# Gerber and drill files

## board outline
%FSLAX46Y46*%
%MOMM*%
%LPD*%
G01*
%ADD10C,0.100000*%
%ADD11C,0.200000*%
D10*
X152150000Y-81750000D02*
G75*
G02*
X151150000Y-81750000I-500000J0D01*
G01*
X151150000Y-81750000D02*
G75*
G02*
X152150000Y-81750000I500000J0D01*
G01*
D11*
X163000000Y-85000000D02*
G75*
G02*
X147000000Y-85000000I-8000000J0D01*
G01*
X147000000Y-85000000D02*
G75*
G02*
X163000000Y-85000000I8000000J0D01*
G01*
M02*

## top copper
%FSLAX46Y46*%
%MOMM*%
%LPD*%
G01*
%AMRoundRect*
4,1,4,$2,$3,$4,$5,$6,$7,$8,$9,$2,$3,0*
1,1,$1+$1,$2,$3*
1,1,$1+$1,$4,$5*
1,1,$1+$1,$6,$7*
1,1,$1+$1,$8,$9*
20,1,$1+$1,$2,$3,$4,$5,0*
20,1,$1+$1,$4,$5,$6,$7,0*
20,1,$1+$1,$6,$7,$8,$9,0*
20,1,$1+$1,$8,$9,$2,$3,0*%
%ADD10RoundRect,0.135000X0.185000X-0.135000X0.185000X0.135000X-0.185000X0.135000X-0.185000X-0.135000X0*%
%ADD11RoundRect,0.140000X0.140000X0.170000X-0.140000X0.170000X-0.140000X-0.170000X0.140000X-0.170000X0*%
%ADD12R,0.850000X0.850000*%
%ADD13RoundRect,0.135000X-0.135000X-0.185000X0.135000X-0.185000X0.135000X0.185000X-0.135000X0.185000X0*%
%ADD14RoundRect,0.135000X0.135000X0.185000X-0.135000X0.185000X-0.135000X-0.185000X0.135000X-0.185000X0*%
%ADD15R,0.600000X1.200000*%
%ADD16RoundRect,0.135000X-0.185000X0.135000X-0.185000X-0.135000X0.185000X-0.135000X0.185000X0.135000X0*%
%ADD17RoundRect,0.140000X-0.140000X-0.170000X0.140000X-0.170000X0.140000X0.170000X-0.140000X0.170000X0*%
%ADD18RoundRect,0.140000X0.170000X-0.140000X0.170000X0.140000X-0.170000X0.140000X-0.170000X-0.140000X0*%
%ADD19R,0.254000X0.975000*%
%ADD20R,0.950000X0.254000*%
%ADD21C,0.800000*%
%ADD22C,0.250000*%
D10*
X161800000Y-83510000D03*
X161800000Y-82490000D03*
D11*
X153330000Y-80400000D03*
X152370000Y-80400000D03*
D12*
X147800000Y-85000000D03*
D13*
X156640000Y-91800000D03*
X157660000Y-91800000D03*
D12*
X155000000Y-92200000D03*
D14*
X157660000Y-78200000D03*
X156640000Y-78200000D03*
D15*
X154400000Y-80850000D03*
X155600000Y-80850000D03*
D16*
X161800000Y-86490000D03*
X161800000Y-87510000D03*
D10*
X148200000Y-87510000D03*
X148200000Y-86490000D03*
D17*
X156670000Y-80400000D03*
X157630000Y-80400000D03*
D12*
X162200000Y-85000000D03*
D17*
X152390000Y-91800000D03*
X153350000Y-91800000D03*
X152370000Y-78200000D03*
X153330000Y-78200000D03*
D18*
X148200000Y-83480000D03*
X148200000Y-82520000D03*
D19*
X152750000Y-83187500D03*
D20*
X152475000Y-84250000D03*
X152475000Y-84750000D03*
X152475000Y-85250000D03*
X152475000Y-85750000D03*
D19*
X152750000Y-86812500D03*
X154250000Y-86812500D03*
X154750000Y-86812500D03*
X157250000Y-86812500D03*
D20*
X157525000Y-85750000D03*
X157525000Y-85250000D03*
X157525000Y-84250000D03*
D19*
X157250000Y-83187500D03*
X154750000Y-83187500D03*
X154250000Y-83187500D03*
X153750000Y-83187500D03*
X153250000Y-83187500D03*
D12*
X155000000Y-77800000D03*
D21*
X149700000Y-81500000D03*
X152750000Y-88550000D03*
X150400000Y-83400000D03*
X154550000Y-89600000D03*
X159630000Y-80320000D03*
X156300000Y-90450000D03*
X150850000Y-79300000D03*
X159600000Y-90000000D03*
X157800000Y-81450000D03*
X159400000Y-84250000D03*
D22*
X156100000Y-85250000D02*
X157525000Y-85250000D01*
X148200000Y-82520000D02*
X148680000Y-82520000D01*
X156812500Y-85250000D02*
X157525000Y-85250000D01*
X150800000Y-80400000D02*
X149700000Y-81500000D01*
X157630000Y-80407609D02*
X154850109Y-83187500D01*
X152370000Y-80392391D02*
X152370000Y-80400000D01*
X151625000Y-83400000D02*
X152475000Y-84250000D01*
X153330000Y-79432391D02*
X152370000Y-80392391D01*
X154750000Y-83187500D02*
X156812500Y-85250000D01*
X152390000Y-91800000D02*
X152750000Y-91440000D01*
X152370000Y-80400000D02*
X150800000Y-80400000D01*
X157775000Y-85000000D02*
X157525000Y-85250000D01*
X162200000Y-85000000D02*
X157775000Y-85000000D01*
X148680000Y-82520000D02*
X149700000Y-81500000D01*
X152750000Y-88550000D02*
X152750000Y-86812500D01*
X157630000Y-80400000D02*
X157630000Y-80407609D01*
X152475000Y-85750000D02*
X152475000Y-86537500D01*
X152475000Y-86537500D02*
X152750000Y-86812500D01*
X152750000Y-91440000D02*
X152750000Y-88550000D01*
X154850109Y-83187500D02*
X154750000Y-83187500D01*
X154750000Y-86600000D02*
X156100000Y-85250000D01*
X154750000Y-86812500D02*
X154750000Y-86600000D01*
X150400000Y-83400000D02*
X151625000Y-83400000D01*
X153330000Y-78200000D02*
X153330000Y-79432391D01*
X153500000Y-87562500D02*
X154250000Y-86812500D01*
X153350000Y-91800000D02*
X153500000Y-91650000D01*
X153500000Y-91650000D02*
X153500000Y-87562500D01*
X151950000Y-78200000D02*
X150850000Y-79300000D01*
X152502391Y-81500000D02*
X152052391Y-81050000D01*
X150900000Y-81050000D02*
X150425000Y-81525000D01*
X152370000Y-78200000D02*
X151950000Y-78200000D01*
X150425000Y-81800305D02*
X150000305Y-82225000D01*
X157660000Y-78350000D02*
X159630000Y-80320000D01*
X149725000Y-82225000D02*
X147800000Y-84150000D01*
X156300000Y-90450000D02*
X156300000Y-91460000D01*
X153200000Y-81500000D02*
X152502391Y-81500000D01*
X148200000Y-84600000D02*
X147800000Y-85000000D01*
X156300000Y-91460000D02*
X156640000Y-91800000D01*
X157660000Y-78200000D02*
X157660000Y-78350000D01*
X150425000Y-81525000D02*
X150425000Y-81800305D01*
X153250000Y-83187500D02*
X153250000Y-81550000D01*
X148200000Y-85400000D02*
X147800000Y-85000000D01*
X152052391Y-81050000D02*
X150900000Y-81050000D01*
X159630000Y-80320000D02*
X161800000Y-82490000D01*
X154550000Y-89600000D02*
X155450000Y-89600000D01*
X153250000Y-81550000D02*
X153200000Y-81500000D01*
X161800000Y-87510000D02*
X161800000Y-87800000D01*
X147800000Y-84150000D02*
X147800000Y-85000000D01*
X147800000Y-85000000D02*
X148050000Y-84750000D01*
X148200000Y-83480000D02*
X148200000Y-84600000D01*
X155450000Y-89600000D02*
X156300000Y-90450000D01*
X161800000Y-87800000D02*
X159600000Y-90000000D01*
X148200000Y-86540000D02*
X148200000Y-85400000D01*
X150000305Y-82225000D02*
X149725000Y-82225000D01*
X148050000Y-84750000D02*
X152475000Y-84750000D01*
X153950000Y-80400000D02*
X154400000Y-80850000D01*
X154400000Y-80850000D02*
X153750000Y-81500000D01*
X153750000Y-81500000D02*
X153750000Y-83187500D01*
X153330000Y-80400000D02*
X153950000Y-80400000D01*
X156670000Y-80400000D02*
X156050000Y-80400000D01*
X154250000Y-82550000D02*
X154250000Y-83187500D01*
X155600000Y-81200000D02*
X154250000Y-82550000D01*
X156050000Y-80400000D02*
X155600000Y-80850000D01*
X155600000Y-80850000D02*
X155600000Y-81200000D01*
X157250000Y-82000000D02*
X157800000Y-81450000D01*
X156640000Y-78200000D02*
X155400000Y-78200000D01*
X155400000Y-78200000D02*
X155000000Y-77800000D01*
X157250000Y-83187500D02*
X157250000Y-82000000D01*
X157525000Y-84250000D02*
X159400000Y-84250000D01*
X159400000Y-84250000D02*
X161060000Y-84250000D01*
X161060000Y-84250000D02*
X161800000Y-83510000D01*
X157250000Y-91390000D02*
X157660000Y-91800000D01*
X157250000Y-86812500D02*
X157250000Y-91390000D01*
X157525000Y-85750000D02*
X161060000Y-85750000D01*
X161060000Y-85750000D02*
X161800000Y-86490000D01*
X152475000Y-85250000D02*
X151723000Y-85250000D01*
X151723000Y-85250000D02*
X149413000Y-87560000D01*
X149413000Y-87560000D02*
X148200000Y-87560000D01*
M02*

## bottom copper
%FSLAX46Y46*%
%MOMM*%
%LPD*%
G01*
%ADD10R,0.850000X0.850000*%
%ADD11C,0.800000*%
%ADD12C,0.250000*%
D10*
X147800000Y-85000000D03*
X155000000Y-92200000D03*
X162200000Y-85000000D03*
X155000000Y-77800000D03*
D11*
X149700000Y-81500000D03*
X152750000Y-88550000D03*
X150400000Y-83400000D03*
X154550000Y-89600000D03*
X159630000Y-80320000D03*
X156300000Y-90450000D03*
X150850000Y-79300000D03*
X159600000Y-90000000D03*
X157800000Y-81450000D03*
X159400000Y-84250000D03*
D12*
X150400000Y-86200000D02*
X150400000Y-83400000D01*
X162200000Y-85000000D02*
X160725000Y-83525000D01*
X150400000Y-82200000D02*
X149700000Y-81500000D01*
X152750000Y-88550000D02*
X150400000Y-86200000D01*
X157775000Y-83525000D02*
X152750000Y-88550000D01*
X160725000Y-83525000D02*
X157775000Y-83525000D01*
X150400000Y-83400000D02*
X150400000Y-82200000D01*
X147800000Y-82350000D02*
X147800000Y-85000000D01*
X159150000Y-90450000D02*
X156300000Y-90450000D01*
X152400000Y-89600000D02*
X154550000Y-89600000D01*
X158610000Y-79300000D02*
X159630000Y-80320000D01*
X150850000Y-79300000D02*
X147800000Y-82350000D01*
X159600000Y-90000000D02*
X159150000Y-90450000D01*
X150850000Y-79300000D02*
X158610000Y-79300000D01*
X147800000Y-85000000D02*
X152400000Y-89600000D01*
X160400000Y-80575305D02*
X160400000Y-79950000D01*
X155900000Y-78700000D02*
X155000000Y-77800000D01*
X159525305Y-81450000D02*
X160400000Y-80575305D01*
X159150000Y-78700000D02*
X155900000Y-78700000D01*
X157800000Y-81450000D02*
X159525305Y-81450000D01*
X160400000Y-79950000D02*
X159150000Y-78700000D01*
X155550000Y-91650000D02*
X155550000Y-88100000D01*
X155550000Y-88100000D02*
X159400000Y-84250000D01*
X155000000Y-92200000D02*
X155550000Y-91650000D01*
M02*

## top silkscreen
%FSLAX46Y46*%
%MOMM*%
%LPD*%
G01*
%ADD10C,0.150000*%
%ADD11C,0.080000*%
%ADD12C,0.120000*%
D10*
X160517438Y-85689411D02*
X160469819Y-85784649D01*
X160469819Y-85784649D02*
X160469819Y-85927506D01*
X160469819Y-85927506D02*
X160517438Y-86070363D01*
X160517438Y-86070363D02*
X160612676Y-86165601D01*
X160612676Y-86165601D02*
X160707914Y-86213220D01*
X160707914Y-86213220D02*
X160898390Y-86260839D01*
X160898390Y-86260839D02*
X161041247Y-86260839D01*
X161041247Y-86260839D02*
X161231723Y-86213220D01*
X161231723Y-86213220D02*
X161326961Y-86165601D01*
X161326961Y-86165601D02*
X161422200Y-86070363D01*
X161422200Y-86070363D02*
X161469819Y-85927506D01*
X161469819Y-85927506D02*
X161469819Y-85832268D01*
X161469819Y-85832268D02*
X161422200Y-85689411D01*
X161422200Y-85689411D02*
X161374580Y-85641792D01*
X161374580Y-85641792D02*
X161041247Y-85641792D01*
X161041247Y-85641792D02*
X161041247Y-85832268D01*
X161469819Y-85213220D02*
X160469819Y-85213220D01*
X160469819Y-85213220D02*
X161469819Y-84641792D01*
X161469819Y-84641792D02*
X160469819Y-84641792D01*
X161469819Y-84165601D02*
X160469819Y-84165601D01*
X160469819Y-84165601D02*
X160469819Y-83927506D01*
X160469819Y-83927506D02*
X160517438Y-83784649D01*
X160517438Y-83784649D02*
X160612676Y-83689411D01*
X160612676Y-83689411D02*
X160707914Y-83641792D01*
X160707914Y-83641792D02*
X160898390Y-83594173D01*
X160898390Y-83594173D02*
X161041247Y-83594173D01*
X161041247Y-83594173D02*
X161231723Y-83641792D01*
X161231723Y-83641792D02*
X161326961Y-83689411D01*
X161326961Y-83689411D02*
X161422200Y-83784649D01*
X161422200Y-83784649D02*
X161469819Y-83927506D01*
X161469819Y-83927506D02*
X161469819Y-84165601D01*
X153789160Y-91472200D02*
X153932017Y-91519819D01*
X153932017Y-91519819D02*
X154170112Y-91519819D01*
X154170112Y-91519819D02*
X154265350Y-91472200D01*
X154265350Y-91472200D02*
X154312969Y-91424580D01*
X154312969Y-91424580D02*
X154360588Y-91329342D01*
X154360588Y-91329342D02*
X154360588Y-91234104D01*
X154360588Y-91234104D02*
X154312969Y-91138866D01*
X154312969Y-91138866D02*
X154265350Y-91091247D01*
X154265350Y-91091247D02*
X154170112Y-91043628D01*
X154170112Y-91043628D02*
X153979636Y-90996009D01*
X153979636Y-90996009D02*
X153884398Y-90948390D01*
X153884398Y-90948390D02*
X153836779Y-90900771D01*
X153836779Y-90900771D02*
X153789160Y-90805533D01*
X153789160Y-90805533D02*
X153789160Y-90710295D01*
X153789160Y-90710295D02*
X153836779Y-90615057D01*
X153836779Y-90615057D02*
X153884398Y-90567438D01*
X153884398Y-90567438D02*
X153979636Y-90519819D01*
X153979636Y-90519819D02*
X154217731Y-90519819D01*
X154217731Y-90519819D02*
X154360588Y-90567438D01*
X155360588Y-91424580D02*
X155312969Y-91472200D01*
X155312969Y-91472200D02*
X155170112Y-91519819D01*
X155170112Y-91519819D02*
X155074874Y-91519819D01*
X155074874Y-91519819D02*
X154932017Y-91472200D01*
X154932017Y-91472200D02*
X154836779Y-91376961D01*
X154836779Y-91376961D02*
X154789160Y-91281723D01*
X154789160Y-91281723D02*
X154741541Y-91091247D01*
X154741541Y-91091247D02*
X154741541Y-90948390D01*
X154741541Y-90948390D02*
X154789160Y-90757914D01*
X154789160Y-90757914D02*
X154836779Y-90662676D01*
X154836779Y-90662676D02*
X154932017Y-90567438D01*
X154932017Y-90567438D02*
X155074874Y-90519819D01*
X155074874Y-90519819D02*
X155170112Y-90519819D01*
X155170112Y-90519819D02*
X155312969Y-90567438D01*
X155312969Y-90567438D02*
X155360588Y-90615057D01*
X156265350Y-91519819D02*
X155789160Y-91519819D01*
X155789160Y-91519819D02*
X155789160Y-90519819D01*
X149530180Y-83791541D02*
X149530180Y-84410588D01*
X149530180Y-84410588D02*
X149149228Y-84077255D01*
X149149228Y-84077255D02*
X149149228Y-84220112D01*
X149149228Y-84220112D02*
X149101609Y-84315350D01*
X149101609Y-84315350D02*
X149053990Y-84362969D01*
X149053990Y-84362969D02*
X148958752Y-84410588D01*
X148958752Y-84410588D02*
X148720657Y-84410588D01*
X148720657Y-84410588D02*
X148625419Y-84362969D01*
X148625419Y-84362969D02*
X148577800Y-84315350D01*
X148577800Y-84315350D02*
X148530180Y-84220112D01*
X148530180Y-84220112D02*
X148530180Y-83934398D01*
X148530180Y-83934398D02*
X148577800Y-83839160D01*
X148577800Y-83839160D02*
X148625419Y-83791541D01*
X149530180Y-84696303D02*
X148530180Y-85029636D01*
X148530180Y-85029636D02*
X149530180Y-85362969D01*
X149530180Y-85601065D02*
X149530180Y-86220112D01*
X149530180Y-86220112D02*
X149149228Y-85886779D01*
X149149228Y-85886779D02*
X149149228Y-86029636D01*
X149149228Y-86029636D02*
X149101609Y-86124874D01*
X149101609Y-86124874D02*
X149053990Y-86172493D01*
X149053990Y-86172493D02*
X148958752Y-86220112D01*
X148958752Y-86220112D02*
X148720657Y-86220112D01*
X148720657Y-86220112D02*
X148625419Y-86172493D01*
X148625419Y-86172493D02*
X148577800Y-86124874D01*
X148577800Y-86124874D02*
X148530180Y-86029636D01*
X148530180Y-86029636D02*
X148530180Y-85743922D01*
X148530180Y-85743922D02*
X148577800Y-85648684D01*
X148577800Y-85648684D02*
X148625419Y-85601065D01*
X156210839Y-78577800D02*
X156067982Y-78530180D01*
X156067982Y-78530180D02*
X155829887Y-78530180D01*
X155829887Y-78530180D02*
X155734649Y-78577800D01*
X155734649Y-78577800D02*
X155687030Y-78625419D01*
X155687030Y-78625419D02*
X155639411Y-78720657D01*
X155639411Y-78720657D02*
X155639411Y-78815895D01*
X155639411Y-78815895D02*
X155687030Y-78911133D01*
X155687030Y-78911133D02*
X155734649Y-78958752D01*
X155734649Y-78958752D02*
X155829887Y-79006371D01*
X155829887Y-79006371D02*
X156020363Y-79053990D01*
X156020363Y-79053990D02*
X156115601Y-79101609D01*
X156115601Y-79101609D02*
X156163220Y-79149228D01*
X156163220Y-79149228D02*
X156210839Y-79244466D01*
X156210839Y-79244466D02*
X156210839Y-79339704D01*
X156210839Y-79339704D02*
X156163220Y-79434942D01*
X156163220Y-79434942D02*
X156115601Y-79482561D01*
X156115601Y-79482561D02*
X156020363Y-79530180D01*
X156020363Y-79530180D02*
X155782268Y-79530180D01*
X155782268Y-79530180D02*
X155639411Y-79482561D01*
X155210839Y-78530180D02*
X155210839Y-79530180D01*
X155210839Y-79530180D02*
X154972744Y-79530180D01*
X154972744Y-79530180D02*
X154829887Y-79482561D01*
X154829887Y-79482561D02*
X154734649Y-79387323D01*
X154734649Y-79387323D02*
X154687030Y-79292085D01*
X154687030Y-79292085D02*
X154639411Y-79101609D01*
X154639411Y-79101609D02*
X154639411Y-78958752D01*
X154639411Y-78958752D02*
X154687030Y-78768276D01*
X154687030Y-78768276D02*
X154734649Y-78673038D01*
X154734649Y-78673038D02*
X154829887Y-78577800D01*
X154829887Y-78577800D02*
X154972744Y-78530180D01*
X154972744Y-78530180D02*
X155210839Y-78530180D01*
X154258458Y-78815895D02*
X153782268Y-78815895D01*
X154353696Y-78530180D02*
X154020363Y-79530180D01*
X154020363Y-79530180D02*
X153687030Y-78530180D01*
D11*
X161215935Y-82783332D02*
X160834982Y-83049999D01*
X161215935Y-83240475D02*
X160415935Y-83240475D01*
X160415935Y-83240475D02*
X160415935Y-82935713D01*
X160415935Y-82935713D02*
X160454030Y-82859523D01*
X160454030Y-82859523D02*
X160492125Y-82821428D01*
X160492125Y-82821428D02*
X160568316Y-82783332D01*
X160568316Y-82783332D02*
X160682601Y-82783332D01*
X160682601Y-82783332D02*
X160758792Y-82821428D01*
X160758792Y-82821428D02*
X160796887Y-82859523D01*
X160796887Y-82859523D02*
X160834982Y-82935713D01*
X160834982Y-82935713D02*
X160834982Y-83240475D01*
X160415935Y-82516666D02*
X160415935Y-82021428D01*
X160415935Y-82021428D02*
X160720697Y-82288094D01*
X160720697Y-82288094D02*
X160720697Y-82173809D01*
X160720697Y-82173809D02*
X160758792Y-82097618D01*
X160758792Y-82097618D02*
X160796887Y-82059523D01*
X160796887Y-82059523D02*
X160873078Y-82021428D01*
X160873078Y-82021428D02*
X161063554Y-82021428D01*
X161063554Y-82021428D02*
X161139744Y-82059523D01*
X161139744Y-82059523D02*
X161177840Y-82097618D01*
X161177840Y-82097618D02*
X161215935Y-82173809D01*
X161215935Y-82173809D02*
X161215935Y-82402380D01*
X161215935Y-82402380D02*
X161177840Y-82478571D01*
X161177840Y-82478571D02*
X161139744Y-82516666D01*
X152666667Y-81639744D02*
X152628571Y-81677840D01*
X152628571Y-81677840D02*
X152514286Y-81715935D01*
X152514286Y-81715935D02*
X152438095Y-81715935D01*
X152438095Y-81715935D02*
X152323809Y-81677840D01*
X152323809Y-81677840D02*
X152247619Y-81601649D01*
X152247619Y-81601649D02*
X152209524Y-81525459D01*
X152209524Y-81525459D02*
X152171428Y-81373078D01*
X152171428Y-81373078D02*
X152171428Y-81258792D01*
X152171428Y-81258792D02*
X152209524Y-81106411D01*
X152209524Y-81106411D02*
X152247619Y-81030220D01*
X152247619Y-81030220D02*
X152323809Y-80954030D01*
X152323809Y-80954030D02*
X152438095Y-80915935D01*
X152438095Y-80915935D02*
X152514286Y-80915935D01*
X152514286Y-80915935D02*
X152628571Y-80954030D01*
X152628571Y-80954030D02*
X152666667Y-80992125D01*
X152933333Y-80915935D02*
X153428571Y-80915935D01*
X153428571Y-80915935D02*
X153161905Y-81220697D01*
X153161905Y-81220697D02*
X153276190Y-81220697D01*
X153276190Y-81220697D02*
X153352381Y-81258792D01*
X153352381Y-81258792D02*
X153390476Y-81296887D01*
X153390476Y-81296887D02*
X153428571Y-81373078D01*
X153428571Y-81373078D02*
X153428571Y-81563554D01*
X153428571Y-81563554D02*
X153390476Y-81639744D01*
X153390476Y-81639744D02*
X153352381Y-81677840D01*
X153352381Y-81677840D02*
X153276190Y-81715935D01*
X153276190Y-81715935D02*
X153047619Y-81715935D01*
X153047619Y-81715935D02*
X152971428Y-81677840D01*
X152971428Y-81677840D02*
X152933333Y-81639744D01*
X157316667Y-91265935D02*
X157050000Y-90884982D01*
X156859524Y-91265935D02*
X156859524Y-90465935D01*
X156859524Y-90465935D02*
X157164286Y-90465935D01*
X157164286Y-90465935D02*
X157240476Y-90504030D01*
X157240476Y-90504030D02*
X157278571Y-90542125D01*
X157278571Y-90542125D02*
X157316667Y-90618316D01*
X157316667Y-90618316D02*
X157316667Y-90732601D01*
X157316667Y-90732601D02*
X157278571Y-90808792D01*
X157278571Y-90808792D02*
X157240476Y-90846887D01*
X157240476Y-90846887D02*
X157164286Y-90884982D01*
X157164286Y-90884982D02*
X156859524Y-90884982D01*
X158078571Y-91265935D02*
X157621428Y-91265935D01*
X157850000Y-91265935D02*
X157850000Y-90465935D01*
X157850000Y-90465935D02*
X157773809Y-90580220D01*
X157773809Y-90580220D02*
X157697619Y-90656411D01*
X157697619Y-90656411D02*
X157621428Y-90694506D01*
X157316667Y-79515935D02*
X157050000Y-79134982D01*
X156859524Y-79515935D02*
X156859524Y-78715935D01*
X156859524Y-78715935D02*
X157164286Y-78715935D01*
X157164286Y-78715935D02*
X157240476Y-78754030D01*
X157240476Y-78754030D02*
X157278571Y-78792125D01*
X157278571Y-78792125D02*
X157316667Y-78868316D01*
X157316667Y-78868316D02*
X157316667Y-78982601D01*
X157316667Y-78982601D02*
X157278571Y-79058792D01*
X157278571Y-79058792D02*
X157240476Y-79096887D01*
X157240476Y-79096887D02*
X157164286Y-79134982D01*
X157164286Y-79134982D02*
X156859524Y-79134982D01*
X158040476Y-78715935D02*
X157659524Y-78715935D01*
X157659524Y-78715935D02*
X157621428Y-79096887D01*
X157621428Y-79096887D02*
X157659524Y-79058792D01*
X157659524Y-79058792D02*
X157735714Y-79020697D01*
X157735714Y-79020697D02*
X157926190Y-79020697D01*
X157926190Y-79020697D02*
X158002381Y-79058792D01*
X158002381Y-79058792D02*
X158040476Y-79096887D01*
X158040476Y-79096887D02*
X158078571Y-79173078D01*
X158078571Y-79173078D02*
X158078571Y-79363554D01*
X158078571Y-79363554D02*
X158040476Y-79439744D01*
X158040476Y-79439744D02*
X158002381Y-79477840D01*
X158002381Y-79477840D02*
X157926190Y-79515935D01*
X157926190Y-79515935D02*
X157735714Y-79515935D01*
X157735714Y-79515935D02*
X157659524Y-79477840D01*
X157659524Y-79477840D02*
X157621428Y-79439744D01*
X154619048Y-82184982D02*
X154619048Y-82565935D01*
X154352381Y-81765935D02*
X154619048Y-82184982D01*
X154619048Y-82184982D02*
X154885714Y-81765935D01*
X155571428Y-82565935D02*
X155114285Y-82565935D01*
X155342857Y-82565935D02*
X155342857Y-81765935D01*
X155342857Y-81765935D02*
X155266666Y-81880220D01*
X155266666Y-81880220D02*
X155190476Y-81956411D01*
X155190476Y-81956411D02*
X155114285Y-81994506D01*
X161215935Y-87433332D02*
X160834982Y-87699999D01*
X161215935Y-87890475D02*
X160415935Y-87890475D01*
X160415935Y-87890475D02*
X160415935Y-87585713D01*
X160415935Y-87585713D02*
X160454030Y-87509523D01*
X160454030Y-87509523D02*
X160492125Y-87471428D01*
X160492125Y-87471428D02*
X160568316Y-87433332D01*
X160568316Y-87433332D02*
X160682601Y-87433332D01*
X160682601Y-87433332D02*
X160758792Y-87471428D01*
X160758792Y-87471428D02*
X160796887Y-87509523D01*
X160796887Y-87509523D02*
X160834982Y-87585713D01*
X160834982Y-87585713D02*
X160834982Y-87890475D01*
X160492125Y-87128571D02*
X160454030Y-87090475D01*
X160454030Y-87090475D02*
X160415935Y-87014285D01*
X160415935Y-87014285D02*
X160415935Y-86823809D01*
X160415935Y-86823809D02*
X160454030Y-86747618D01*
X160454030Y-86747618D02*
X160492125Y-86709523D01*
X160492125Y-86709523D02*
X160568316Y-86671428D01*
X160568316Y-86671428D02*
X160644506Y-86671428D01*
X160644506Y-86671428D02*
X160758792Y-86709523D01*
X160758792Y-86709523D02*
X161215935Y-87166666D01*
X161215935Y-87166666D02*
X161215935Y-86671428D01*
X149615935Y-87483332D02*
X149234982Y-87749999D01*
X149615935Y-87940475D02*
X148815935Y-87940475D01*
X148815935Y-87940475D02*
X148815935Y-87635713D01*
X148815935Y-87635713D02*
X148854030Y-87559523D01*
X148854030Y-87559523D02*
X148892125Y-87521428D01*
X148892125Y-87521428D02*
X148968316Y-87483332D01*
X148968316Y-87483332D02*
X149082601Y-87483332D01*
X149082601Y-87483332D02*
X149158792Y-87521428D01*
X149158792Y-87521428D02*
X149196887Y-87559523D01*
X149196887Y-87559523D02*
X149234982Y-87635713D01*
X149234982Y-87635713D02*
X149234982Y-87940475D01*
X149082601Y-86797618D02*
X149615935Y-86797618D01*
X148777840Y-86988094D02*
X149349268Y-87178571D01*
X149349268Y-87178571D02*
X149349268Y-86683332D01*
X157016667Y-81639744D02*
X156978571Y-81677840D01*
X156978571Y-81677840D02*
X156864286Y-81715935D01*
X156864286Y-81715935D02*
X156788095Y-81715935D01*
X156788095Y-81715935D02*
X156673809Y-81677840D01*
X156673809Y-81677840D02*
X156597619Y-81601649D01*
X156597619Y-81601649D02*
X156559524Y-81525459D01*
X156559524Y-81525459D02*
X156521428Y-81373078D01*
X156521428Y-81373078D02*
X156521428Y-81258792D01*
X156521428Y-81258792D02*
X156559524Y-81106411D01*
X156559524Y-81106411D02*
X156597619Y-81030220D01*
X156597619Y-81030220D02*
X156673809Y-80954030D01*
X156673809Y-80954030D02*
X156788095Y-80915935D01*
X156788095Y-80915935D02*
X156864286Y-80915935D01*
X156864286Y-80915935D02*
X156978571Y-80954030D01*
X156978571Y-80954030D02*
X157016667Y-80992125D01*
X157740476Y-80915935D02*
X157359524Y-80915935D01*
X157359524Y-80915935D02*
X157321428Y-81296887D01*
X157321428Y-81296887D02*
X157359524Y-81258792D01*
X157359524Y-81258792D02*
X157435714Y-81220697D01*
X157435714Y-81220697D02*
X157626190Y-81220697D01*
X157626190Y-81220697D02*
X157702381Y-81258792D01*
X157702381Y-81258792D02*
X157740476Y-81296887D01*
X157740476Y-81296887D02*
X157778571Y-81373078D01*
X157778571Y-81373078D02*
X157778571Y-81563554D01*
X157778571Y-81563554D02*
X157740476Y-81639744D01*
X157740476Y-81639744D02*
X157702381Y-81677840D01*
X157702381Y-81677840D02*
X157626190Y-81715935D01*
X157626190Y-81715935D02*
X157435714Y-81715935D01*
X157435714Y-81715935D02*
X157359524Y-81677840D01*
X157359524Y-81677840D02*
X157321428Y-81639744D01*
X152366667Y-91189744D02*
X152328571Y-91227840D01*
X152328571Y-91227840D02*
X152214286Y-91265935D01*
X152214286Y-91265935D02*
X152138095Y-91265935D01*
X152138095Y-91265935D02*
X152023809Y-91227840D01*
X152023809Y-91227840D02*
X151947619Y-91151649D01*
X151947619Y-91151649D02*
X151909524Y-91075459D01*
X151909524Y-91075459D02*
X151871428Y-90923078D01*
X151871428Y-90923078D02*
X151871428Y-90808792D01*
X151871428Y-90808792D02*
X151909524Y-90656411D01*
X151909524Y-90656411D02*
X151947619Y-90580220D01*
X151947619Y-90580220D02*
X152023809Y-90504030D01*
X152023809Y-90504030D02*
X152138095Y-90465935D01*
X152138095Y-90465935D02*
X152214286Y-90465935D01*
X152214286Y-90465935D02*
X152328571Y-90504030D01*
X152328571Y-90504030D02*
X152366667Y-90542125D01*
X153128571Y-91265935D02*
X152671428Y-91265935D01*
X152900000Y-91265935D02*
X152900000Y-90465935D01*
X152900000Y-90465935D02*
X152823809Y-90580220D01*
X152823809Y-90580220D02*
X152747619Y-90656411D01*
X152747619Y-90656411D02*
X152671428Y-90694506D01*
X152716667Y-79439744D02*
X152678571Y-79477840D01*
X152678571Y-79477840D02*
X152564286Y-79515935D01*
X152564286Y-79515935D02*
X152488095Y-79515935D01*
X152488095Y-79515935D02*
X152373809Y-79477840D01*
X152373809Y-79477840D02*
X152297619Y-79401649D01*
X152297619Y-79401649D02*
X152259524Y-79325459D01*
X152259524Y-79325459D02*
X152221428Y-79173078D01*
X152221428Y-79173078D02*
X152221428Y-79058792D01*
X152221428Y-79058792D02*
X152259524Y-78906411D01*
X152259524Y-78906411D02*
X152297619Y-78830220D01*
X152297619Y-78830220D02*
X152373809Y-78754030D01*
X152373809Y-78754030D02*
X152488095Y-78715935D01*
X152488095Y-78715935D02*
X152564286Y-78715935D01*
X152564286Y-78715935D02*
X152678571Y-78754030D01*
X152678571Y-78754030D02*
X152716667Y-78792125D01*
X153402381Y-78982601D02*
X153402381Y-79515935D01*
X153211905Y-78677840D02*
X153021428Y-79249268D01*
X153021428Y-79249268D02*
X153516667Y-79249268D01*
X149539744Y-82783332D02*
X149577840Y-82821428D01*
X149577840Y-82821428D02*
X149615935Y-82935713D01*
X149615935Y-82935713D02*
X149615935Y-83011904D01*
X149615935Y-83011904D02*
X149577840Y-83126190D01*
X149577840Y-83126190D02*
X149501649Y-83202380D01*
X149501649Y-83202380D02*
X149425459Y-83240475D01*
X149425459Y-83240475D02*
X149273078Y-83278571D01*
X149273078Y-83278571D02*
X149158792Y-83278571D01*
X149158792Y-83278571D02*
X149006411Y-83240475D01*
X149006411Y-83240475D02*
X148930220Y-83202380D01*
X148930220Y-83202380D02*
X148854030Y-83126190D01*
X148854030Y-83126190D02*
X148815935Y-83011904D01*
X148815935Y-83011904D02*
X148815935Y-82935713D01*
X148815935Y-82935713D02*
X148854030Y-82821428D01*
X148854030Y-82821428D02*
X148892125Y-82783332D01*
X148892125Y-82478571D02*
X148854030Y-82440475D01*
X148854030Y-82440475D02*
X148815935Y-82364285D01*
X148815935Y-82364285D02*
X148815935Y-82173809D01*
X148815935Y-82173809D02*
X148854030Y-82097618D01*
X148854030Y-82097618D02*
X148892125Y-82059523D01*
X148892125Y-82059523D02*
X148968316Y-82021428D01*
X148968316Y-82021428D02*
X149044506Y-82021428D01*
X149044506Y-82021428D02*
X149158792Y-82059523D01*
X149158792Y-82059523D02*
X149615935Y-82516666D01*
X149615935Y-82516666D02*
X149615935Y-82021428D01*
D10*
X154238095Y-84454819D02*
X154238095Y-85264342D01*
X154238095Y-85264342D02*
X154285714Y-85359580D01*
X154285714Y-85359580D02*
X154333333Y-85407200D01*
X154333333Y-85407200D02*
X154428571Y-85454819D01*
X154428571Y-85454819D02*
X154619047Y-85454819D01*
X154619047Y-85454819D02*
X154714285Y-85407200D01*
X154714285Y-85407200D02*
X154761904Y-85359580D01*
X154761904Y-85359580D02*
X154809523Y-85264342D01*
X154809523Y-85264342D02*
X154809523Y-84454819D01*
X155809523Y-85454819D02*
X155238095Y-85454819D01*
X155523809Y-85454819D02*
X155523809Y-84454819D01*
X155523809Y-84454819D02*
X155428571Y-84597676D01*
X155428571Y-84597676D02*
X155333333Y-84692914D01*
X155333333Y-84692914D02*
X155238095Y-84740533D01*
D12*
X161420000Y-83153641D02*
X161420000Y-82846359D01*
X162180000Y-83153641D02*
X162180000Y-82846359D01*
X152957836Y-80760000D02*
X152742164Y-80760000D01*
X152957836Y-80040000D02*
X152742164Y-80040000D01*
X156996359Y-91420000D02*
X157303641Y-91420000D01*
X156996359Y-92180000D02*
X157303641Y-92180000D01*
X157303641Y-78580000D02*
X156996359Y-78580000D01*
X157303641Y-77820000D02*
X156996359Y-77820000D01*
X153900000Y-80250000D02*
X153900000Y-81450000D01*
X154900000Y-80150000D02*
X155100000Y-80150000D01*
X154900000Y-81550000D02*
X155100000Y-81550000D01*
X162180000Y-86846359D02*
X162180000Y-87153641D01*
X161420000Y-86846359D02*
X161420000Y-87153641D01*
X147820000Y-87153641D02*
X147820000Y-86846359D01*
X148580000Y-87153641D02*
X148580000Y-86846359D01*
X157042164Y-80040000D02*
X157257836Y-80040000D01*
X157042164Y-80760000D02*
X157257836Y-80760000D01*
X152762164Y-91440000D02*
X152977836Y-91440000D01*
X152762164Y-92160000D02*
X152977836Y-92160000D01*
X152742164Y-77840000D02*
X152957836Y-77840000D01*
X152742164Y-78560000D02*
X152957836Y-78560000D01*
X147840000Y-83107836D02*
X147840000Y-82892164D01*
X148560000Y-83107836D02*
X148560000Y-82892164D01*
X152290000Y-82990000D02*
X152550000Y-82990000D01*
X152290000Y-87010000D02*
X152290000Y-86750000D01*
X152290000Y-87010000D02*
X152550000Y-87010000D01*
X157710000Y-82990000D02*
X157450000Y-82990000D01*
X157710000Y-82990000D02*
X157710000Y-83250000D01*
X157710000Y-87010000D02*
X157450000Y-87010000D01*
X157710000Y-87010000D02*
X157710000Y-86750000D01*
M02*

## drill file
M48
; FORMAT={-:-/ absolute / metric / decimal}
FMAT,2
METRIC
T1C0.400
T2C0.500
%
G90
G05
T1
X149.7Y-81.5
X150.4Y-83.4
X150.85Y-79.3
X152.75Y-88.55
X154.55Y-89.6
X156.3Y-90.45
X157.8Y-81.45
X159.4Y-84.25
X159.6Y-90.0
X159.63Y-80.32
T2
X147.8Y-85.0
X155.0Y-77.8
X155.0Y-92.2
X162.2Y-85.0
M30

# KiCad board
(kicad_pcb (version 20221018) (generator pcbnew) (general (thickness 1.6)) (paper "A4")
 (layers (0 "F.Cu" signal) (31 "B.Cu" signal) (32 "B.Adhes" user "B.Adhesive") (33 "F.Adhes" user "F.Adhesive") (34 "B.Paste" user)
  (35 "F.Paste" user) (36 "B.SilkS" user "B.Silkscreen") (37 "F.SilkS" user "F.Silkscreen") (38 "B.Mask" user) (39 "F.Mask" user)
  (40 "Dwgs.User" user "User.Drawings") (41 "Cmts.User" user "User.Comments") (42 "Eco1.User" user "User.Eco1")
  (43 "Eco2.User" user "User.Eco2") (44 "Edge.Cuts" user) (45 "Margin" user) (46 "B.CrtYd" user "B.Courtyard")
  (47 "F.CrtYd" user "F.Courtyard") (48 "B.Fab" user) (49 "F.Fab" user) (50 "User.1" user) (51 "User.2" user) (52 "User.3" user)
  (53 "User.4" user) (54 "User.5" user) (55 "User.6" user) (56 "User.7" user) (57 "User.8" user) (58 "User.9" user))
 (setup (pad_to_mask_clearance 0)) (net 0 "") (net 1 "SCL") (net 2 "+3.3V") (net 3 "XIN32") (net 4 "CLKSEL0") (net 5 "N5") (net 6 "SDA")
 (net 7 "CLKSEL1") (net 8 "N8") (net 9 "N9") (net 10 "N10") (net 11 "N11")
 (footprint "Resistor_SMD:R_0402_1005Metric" (layer "F.Cu") (at 161.8 83 90)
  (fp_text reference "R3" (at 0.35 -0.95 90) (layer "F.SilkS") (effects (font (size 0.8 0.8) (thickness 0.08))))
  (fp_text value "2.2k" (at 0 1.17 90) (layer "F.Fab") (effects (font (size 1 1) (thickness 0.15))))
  (fp_line (start -0.153641 -0.38) (end 0.153641 -0.38) (stroke (width 0.12) (type solid)) (layer "F.SilkS"))
  (fp_line (start -0.153641 0.38) (end 0.153641 0.38) (stroke (width 0.12) (type solid)) (layer "F.SilkS"))
  (pad "1" smd roundrect (at -0.51 0 90) (size 0.54 0.64) (layers "F.Cu" "F.Paste" "F.Mask") (roundrect_rratio 0.25) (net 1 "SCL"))
  (pad "2" smd roundrect (at 0.51 0 90) (size 0.54 0.64) (layers "F.Cu" "F.Paste" "F.Mask") (roundrect_rratio 0.25) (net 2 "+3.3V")))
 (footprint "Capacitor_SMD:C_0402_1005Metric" (layer "F.Cu") (at 152.85 80.4 180)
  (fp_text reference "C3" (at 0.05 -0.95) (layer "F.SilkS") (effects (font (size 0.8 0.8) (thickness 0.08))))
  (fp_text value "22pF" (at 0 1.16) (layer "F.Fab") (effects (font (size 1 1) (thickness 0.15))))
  (fp_line (start -0.107836 -0.36) (end 0.107836 -0.36) (stroke (width 0.12) (type solid)) (layer "F.SilkS"))
  (fp_line (start -0.107836 0.36) (end 0.107836 0.36) (stroke (width 0.12) (type solid)) (layer "F.SilkS"))
  (pad "1" smd roundrect (at -0.48 0 180) (size 0.56 0.62) (layers "F.Cu" "F.Paste" "F.Mask") (roundrect_rratio 0.25) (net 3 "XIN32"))
  (pad "2" smd roundrect (at 0.48 0 180) (size 0.56 0.62) (layers "F.Cu" "F.Paste" "F.Mask") (roundrect_rratio 0.25) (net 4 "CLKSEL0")))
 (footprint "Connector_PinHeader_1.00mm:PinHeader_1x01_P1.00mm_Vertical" (layer "F.Cu") (at 147.8 85)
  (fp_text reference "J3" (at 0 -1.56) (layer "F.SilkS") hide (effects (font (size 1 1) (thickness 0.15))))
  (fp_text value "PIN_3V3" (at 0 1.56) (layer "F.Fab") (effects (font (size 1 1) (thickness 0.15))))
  (pad "1" thru_hole rect (at 0 0) (size 0.85 0.85) (drill 0.5) (layers "*.Cu" "*.Mask") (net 2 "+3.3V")))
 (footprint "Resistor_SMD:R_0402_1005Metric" (layer "F.Cu") (at 157.15 91.8)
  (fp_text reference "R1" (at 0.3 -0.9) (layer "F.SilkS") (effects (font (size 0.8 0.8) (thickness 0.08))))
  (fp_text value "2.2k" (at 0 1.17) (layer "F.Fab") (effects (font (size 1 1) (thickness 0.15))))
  (fp_line (start -0.153641 -0.38) (end 0.153641 -0.38) (stroke (width 0.12) (type solid)) (layer "F.SilkS"))
  (fp_line (start -0.153641 0.38) (end 0.153641 0.38) (stroke (width 0.12) (type solid)) (layer "F.SilkS"))
  (pad "1" smd roundrect (at -0.51 0) (size 0.54 0.64) (layers "F.Cu" "F.Paste" "F.Mask") (roundrect_rratio 0.25) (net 2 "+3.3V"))
  (pad "2" smd roundrect (at 0.51 0) (size 0.54 0.64) (layers "F.Cu" "F.Paste" "F.Mask") (roundrect_rratio 0.25) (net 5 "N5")))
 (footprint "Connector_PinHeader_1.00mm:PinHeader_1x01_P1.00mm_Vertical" (layer "F.Cu") (at 155 92.2)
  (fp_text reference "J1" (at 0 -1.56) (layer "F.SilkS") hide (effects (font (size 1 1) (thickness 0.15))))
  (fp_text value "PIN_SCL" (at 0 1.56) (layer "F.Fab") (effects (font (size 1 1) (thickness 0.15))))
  (pad "1" thru_hole rect (at 0 0) (size 0.85 0.85) (drill 0.5) (layers "*.Cu" "*.Mask") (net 1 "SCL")))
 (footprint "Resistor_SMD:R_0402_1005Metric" (layer "F.Cu") (at 157.15 78.2 180)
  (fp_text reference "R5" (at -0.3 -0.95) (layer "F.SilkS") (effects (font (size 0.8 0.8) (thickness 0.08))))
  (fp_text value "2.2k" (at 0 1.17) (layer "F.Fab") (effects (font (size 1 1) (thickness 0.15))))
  (fp_line (start -0.153641 -0.38) (end 0.153641 -0.38) (stroke (width 0.12) (type solid)) (layer "F.SilkS"))
  (fp_line (start -0.153641 0.38) (end 0.153641 0.38) (stroke (width 0.12) (type solid)) (layer "F.SilkS"))
  (pad "1" smd roundrect (at -0.51 0 180) (size 0.54 0.64) (layers "F.Cu" "F.Paste" "F.Mask") (roundrect_rratio 0.25) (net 2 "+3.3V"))
  (pad "2" smd roundrect (at 0.51 0 180) (size 0.54 0.64) (layers "F.Cu" "F.Paste" "F.Mask") (roundrect_rratio 0.25) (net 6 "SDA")))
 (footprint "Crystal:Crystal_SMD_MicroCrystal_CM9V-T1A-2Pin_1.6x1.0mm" (layer "F.Cu") (at 155 80.85)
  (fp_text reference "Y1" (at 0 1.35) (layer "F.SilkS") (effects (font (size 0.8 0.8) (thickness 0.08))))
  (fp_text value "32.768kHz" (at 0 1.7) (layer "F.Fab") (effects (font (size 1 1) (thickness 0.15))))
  (fp_line (start -1.1 -0.6) (end -1.1 0.6) (stroke (width 0.12) (type solid)) (layer "F.SilkS"))
  (fp_line (start -0.1 -0.7) (end 0.1 -0.7) (stroke (width 0.12) (type solid)) (layer "F.SilkS"))
  (fp_line (start -0.1 0.7) (end 0.1 0.7) (stroke (width 0.12) (type solid)) (layer "F.SilkS"))
  (pad "1" smd rect (at -0.6 0) (size 0.6 1.2) (layers "F.Cu" "F.Paste" "F.Mask") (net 3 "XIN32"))
  (pad "2" smd rect (at 0.6 0) (size 0.6 1.2) (layers "F.Cu" "F.Paste" "F.Mask") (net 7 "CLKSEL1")))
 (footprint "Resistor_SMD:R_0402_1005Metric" (layer "F.Cu") (at 161.8 87 -90)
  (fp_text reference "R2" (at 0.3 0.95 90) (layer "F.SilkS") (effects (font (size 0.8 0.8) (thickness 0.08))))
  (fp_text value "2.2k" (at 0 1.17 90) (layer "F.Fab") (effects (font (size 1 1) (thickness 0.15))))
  (fp_line (start -0.153641 -0.38) (end 0.153641 -0.38) (stroke (width 0.12) (type solid)) (layer "F.SilkS"))
  (fp_line (start -0.153641 0.38) (end 0.153641 0.38) (stroke (width 0.12) (type solid)) (layer "F.SilkS"))
  (pad "1" smd roundrect (at -0.51 0 270) (size 0.54 0.64) (layers "F.Cu" "F.Paste" "F.Mask") (roundrect_rratio 0.25) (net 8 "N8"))
  (pad "2" smd roundrect (at 0.51 0 270) (size 0.54 0.64) (layers "F.Cu" "F.Paste" "F.Mask") (roundrect_rratio 0.25) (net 2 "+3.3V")))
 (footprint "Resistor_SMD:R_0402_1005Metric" (layer "F.Cu") (at 148.2 87 90)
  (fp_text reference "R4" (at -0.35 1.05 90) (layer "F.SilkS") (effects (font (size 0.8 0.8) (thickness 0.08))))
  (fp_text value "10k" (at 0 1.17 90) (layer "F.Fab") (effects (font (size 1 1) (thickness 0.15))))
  (fp_line (start -0.153641 -0.38) (end 0.153641 -0.38) (stroke (width 0.12) (type solid)) (layer "F.SilkS"))
  (fp_line (start -0.153641 0.38) (end 0.153641 0.38) (stroke (width 0.12) (type solid)) (layer "F.SilkS"))
  (pad "1" smd roundrect (at -0.51 0 90) (size 0.54 0.64) (layers "F.Cu" "F.Paste" "F.Mask") (roundrect_rratio 0.25) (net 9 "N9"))
  (pad "2" smd roundrect (at 0.51 0 90) (size 0.54 0.64) (layers "F.Cu" "F.Paste" "F.Mask") (roundrect_rratio 0.25) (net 2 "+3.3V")))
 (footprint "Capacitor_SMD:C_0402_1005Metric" (layer "F.Cu") (at 157.15 80.4)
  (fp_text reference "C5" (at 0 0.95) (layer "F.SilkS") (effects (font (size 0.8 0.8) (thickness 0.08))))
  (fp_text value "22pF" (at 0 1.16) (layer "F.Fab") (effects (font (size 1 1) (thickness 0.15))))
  (fp_line (start -0.107836 -0.36) (end 0.107836 -0.36) (stroke (width 0.12) (type solid)) (layer "F.SilkS"))
  (fp_line (start -0.107836 0.36) (end 0.107836 0.36) (stroke (width 0.12) (type solid)) (layer "F.SilkS"))
  (pad "1" smd roundrect (at -0.48 0) (size 0.56 0.62) (layers "F.Cu" "F.Paste" "F.Mask") (roundrect_rratio 0.25) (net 7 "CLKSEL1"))
  (pad "2" smd roundrect (at 0.48 0) (size 0.56 0.62) (layers "F.Cu" "F.Paste" "F.Mask") (roundrect_rratio 0.25) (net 4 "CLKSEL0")))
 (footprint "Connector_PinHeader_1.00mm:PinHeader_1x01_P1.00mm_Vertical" (layer "F.Cu") (at 162.2 85)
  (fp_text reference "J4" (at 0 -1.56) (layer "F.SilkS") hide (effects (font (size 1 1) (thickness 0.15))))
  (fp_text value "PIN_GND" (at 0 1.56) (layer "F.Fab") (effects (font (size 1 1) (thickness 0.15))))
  (pad "1" thru_hole rect (at 0 0) (size 0.85 0.85) (drill 0.5) (layers "*.Cu" "*.Mask") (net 4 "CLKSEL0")))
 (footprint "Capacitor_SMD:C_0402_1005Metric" (layer "F.Cu") (at 152.87 91.8)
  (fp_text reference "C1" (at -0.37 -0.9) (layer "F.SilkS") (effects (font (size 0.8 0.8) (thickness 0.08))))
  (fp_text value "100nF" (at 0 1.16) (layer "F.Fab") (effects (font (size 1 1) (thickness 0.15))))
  (fp_line (start -0.107836 -0.36) (end 0.107836 -0.36) (stroke (width 0.12) (type solid)) (layer "F.SilkS"))
  (fp_line (start -0.107836 0.36) (end 0.107836 0.36) (stroke (width 0.12) (type solid)) (layer "F.SilkS"))
  (pad "1" smd roundrect (at -0.48 0) (size 0.56 0.62) (layers "F.Cu" "F.Paste" "F.Mask") (roundrect_rratio 0.25) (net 4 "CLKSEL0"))
  (pad "2" smd roundrect (at 0.48 0) (size 0.56 0.62) (layers "F.Cu" "F.Paste" "F.Mask") (roundrect_rratio 0.25) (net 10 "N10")))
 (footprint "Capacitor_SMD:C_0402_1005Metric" (layer "F.Cu") (at 152.85 78.2)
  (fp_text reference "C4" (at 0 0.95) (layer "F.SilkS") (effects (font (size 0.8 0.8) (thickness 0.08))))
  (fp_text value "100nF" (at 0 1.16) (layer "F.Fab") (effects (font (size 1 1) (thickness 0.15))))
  (fp_line (start -0.107836 -0.36) (end 0.107836 -0.36) (stroke (width 0.12) (type solid)) (layer "F.SilkS"))
  (fp_line (start -0.107836 0.36) (end 0.107836 0.36) (stroke (width 0.12) (type solid)) (layer "F.SilkS"))
  (pad "1" smd roundrect (at -0.48 0) (size 0.56 0.62) (layers "F.Cu" "F.Paste" "F.Mask") (roundrect_rratio 0.25) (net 2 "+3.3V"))
  (pad "2" smd roundrect (at 0.48 0) (size 0.56 0.62) (layers "F.Cu" "F.Paste" "F.Mask") (roundrect_rratio 0.25) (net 4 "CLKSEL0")))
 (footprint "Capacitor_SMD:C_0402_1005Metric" (layer "F.Cu") (at 148.2 83 90)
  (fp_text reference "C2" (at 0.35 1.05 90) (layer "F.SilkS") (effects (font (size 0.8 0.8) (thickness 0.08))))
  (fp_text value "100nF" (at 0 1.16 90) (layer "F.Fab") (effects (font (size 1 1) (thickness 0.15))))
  (fp_line (start -0.107836 -0.36) (end 0.107836 -0.36) (stroke (width 0.12) (type solid)) (layer "F.SilkS"))
  (fp_line (start -0.107836 0.36) (end 0.107836 0.36) (stroke (width 0.12) (type solid)) (layer "F.SilkS"))
  (pad "1" smd roundrect (at -0.48 0 90) (size 0.56 0.62) (layers "F.Cu" "F.Paste" "F.Mask") (roundrect_rratio 0.25) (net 2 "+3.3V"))
  (pad "2" smd roundrect (at 0.48 0 90) (size 0.56 0.62) (layers "F.Cu" "F.Paste" "F.Mask") (roundrect_rratio 0.25) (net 4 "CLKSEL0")))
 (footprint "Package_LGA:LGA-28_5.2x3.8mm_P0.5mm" (layer "F.Cu") (at 155 85)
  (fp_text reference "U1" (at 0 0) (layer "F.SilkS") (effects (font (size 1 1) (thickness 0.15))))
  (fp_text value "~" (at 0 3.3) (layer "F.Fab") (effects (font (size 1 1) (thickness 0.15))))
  (fp_line (start -2.71 -2.01) (end -2.45 -2.01) (stroke (width 0.12) (type solid)) (layer "F.SilkS"))
  (fp_line (start -2.71 2.01) (end -2.71 1.75) (stroke (width 0.12) (type solid)) (layer "F.SilkS"))
  (fp_line (start -2.71 2.01) (end -2.45 2.01) (stroke (width 0.12) (type solid)) (layer "F.SilkS"))
  (fp_line (start 2.71 -2.01) (end 2.45 -2.01) (stroke (width 0.12) (type solid)) (layer "F.SilkS"))
  (fp_line (start 2.71 -2.01) (end 2.71 -1.75) (stroke (width 0.12) (type solid)) (layer "F.SilkS"))
  (fp_line (start 2.71 2.01) (end 2.45 2.01) (stroke (width 0.12) (type solid)) (layer "F.SilkS"))
  (fp_line (start 2.71 2.01) (end 2.71 1.75) (stroke (width 0.12) (type solid)) (layer "F.SilkS"))
  (pad "1" smd rect (at -2.25 -1.8125) (size 0.254 0.975) (layers "F.Cu" "F.Paste" "F.Mask") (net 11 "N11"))
  (pad "2" smd rect (at -2.525 -0.75 90) (size 0.254 0.95) (layers "F.Cu" "F.Paste" "F.Mask") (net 4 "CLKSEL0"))
  (pad "3" smd rect (at -2.525 -0.25 90) (size 0.254 0.95) (layers "F.Cu" "F.Paste" "F.Mask") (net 2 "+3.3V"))
  (pad "4" smd rect (at -2.525 0.25 90) (size 0.254 0.95) (layers "F.Cu" "F.Paste" "F.Mask") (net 9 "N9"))
  (pad "5" smd rect (at -2.525 0.75 90) (size 0.254 0.95) (layers "F.Cu" "F.Paste" "F.Mask") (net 4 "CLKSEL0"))
  (pad "6" smd rect (at -2.25 1.8125) (size 0.254 0.975) (layers "F.Cu" "F.Paste" "F.Mask") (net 4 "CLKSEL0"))
  (pad "9" smd rect (at -0.75 1.8125) (size 0.254 0.975) (layers "F.Cu" "F.Paste" "F.Mask") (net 10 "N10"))
  (pad "10" smd rect (at -0.25 1.8125) (size 0.254 0.975) (layers "F.Cu" "F.Paste" "F.Mask") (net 4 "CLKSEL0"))
  (pad "15" smd rect (at 2.25 1.8125) (size 0.254 0.975) (layers "F.Cu" "F.Paste" "F.Mask") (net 5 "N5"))
  (pad "16" smd rect (at 2.525 0.75 90) (size 0.254 0.95) (layers "F.Cu" "F.Paste" "F.Mask") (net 8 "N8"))
  (pad "17" smd rect (at 2.525 0.25 90) (size 0.254 0.95) (layers "F.Cu" "F.Paste" "F.Mask") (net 4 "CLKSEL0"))
  (pad "19" smd rect (at 2.525 -0.75 90) (size 0.254 0.95) (layers "F.Cu" "F.Paste" "F.Mask") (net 1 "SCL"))
  (pad "20" smd rect (at 2.25 -1.8125) (size 0.254 0.975) (layers "F.Cu" "F.Paste" "F.Mask") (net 6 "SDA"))
  (pad "25" smd rect (at -0.25 -1.8125) (size 0.254 0.975) (layers "F.Cu" "F.Paste" "F.Mask") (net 4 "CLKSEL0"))
  (pad "26" smd rect (at -0.75 -1.8125) (size 0.254 0.975) (layers "F.Cu" "F.Paste" "F.Mask") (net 7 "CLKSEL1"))
  (pad "27" smd rect (at -1.25 -1.8125) (size 0.254 0.975) (layers "F.Cu" "F.Paste" "F.Mask") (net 3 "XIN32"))
  (pad "28" smd rect (at -1.75 -1.8125) (size 0.254 0.975) (layers "F.Cu" "F.Paste" "F.Mask") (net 2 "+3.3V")))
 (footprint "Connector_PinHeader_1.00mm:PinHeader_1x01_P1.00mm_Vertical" (layer "F.Cu") (at 155 77.8)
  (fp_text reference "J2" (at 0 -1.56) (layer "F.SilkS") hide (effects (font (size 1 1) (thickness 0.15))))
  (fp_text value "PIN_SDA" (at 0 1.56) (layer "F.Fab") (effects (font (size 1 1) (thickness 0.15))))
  (pad "1" thru_hole rect (at 0 0) (size 0.85 0.85) (drill 0.5) (layers "*.Cu" "*.Mask") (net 6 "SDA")))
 (gr_circle (center 151.65 81.75) (end 152.15 81.75) (stroke (width 0.1) (type default)) (fill none) (layer "Edge.Cuts"))
 (gr_circle (center 155 85) (end 163 85) (stroke (width 0.2) (type default)) (fill none) (layer "Edge.Cuts"))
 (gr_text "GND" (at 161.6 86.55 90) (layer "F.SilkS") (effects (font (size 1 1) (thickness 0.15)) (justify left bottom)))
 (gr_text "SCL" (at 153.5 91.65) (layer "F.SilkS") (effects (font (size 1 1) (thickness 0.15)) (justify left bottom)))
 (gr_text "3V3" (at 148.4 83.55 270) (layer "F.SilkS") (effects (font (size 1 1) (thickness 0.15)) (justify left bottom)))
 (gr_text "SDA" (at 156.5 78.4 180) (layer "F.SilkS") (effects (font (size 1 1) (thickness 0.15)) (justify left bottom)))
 (segment (start 156.1 85.25) (end 157.525 85.25) (width 0.25) (layer "F.Cu") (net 4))
 (segment (start 148.2 82.52) (end 148.68 82.52) (width 0.25) (layer "F.Cu") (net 4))
 (segment (start 156.8125 85.25) (end 157.525 85.25) (width 0.25) (layer "F.Cu") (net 4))
 (segment (start 150.8 80.4) (end 149.7 81.5) (width 0.25) (layer "F.Cu") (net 4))
 (segment (start 157.63 80.407609) (end 154.850109 83.1875) (width 0.25) (layer "F.Cu") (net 4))
 (segment (start 152.37 80.392391) (end 152.37 80.4) (width 0.25) (layer "F.Cu") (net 4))
 (segment (start 151.625 83.4) (end 152.475 84.25) (width 0.25) (layer "F.Cu") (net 4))
 (segment (start 153.33 79.432391) (end 152.37 80.392391) (width 0.25) (layer "F.Cu") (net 4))
 (segment (start 154.75 83.1875) (end 156.8125 85.25) (width 0.25) (layer "F.Cu") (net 4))
 (segment (start 152.39 91.8) (end 152.75 91.44) (width 0.25) (layer "F.Cu") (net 4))
 (segment (start 152.37 80.4) (end 150.8 80.4) (width 0.25) (layer "F.Cu") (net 4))
 (segment (start 157.775 85) (end 157.525 85.25) (width 0.25) (layer "F.Cu") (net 4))
 (segment (start 162.2 85) (end 157.775 85) (width 0.25) (layer "F.Cu") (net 4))
 (segment (start 148.68 82.52) (end 149.7 81.5) (width 0.25) (layer "F.Cu") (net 4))
 (segment (start 152.75 88.55) (end 152.75 86.8125) (width 0.25) (layer "F.Cu") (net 4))
 (segment (start 157.63 80.4) (end 157.63 80.407609) (width 0.25) (layer "F.Cu") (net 4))
 (segment (start 152.475 85.75) (end 152.475 86.5375) (width 0.25) (layer "F.Cu") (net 4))
 (segment (start 152.475 86.5375) (end 152.75 86.8125) (width 0.25) (layer "F.Cu") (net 4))
 (segment (start 152.75 91.44) (end 152.75 88.55) (width 0.25) (layer "F.Cu") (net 4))
 (segment (start 154.850109 83.1875) (end 154.75 83.1875) (width 0.25) (layer "F.Cu") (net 4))
 (segment (start 154.75 86.6) (end 156.1 85.25) (width 0.25) (layer "F.Cu") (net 4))
 (segment (start 154.75 86.8125) (end 154.75 86.6) (width 0.25) (layer "F.Cu") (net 4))
 (segment (start 150.4 83.4) (end 151.625 83.4) (width 0.25) (layer "F.Cu") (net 4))
 (segment (start 153.33 78.2) (end 153.33 79.432391) (width 0.25) (layer "F.Cu") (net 4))
 (via (at 149.7 81.5) (size 0.8) (drill 0.4) (layers "F.Cu" "B.Cu") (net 4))
 (via (at 152.75 88.55) (size 0.8) (drill 0.4) (layers "F.Cu" "B.Cu") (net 4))
 (via (at 150.4 83.4) (size 0.8) (drill 0.4) (layers "F.Cu" "B.Cu") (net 4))
 (segment (start 150.4 86.2) (end 150.4 83.4) (width 0.25) (layer "B.Cu") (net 4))
 (segment (start 162.2 85) (end 160.725 83.525) (width 0.25) (layer "B.Cu") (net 4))
 (segment (start 150.4 82.2) (end 149.7 81.5) (width 0.25) (layer "B.Cu") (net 4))
 (segment (start 152.75 88.55) (end 150.4 86.2) (width 0.25) (layer "B.Cu") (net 4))
 (segment (start 157.775 83.525) (end 152.75 88.55) (width 0.25) (layer "B.Cu") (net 4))
 (segment (start 160.725 83.525) (end 157.775 83.525) (width 0.25) (layer "B.Cu") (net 4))
 (segment (start 150.4 83.4) (end 150.4 82.2) (width 0.25) (layer "B.Cu") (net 4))
 (segment (start 153.5 87.5625) (end 154.25 86.8125) (width 0.25) (layer "F.Cu") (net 10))
 (segment (start 153.35 91.8) (end 153.5 91.65) (width 0.25) (layer "F.Cu") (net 10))
 (segment (start 153.5 91.65) (end 153.5 87.5625) (width 0.25) (layer "F.Cu") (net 10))
 (segment (start 151.95 78.2) (end 150.85 79.3) (width 0.25) (layer "F.Cu") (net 2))
 (segment (start 152.502391 81.5) (end 152.052391 81.05) (width 0.25) (layer "F.Cu") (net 2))
 (segment (start 150.9 81.05) (end 150.425 81.525) (width 0.25) (layer "F.Cu") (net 2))
 (segment (start 152.37 78.2) (end 151.95 78.2) (width 0.25) (layer "F.Cu") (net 2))
 (segment (start 150.425 81.800305) (end 150.000305 82.225) (width 0.25) (layer "F.Cu") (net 2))
 (segment (start 157.66 78.35) (end 159.63 80.32) (width 0.25) (layer "F.Cu") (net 2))
 (segment (start 149.725 82.225) (end 147.8 84.15) (width 0.25) (layer "F.Cu") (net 2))
 (segment (start 156.3 90.45) (end 156.3 91.46) (width 0.25) (layer "F.Cu") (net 2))
 (segment (start 153.2 81.5) (end 152.502391 81.5) (width 0.25) (layer "F.Cu") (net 2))
 (segment (start 148.2 84.6) (end 147.8 85) (width 0.25) (layer "F.Cu") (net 2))
 (segment (start 156.3 91.46) (end 156.64 91.8) (width 0.25) (layer "F.Cu") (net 2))
 (segment (start 157.66 78.2) (end 157.66 78.35) (width 0.25) (layer "F.Cu") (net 2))
 (segment (start 150.425 81.525) (end 150.425 81.800305) (width 0.25) (layer "F.Cu") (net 2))
 (segment (start 153.25 83.1875) (end 153.25 81.55) (width 0.25) (layer "F.Cu") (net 2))
 (segment (start 148.2 85.4) (end 147.8 85) (width 0.25) (layer "F.Cu") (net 2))
 (segment (start 152.052391 81.05) (end 150.9 81.05) (width 0.25) (layer "F.Cu") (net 2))
 (segment (start 159.63 80.32) (end 161.8 82.49) (width 0.25) (layer "F.Cu") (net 2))
 (segment (start 154.55 89.6) (end 155.45 89.6) (width 0.25) (layer "F.Cu") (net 2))
 (segment (start 153.25 81.55) (end 153.2 81.5) (width 0.25) (layer "F.Cu") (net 2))
 (segment (start 161.8 87.51) (end 161.8 87.8) (width 0.25) (layer "F.Cu") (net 2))
 (segment (start 147.8 84.15) (end 147.8 85) (width 0.25) (layer "F.Cu") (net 2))
 (segment (start 147.8 85) (end 148.05 84.75) (width 0.25) (layer "F.Cu") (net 2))
 (segment (start 148.2 83.48) (end 148.2 84.6) (width 0.25) (layer "F.Cu") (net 2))
 (segment (start 155.45 89.6) (end 156.3 90.45) (width 0.25) (layer "F.Cu") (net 2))
 (segment (start 161.8 87.8) (end 159.6 90) (width 0.25) (layer "F.Cu") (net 2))
 (segment (start 148.2 86.54) (end 148.2 85.4) (width 0.25) (layer "F.Cu") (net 2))
 (segment (start 150.000305 82.225) (end 149.725 82.225) (width 0.25) (layer "F.Cu") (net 2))
 (segment (start 148.05 84.75) (end 152.475 84.75) (width 0.25) (layer "F.Cu") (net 2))
 (via (at 154.55 89.6) (size 0.8) (drill 0.4) (layers "F.Cu" "B.Cu") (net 2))
 (via (at 159.63 80.32) (size 0.8) (drill 0.4) (layers "F.Cu" "B.Cu") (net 2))
 (via (at 156.3 90.45) (size 0.8) (drill 0.4) (layers "F.Cu" "B.Cu") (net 2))
 (via (at 150.85 79.3) (size 0.8) (drill 0.4) (layers "F.Cu" "B.Cu") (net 2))
 (via (at 159.6 90) (size 0.8) (drill 0.4) (layers "F.Cu" "B.Cu") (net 2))
 (segment (start 147.8 82.35) (end 147.8 85) (width 0.25) (layer "B.Cu") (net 2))
 (segment (start 159.15 90.45) (end 156.3 90.45) (width 0.25) (layer "B.Cu") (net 2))
 (segment (start 152.4 89.6) (end 154.55 89.6) (width 0.25) (layer "B.Cu") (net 2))
 (segment (start 158.61 79.3) (end 159.63 80.32) (width 0.25) (layer "B.Cu") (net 2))
 (segment (start 150.85 79.3) (end 147.8 82.35) (width 0.25) (layer "B.Cu") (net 2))
 (segment (start 159.6 90) (end 159.15 90.45) (width 0.25) (layer "B.Cu") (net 2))
 (segment (start 150.85 79.3) (end 158.61 79.3) (width 0.25) (layer "B.Cu") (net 2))
 (segment (start 147.8 85) (end 152.4 89.6) (width 0.25) (layer "B.Cu") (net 2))
 (segment (start 153.95 80.4) (end 154.4 80.85) (width 0.25) (layer "F.Cu") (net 3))
 (segment (start 154.4 80.85) (end 153.75 81.5) (width 0.25) (layer "F.Cu") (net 3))
 (segment (start 153.75 81.5) (end 153.75 83.1875) (width 0.25) (layer "F.Cu") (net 3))
 (segment (start 153.33 80.4) (end 153.95 80.4) (width 0.25) (layer "F.Cu") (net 3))
 (segment (start 156.67 80.4) (end 156.05 80.4) (width 0.25) (layer "F.Cu") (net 7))
 (segment (start 154.25 82.55) (end 154.25 83.1875) (width 0.25) (layer "F.Cu") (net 7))
 (segment (start 155.6 81.2) (end 154.25 82.55) (width 0.25) (layer "F.Cu") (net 7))
 (segment (start 156.05 80.4) (end 155.6 80.85) (width 0.25) (layer "F.Cu") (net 7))
 (segment (start 155.6 80.85) (end 155.6 81.2) (width 0.25) (layer "F.Cu") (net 7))
 (segment (start 157.25 82) (end 157.8 81.45) (width 0.25) (layer "F.Cu") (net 6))
 (segment (start 156.64 78.2) (end 155.4 78.2) (width 0.25) (layer "F.Cu") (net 6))
 (segment (start 155.4 78.2) (end 155 77.8) (width 0.25) (layer "F.Cu") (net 6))
 (segment (start 157.25 83.1875) (end 157.25 82) (width 0.25) (layer "F.Cu") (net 6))
 (via (at 157.8 81.45) (size 0.8) (drill 0.4) (layers "F.Cu" "B.Cu") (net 6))
 (segment (start 160.4 80.575305) (end 160.4 79.95) (width 0.25) (layer "B.Cu") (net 6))
 (segment (start 155.9 78.7) (end 155 77.8) (width 0.25) (layer "B.Cu") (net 6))
 (segment (start 159.525305 81.45) (end 160.4 80.575305) (width 0.25) (layer "B.Cu") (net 6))
 (segment (start 159.15 78.7) (end 155.9 78.7) (width 0.25) (layer "B.Cu") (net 6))
 (segment (start 157.8 81.45) (end 159.525305 81.45) (width 0.25) (layer "B.Cu") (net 6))
 (segment (start 160.4 79.95) (end 159.15 78.7) (width 0.25) (layer "B.Cu") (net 6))
 (segment (start 157.525 84.25) (end 159.4 84.25) (width 0.25) (layer "F.Cu") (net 1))
 (segment (start 159.4 84.25) (end 161.06 84.25) (width 0.25) (layer "F.Cu") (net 1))
 (segment (start 161.06 84.25) (end 161.8 83.51) (width 0.25) (layer "F.Cu") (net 1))
 (via (at 159.4 84.25) (size 0.8) (drill 0.4) (layers "F.Cu" "B.Cu") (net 1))
 (segment (start 155.55 91.65) (end 155.55 88.1) (width 0.25) (layer "B.Cu") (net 1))
 (segment (start 155.55 88.1) (end 159.4 84.25) (width 0.25) (layer "B.Cu") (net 1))
 (segment (start 155 92.2) (end 155.55 91.65) (width 0.25) (layer "B.Cu") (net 1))
 (segment (start 157.25 91.39) (end 157.66 91.8) (width 0.25) (layer "F.Cu") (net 5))
 (segment (start 157.25 86.8125) (end 157.25 91.39) (width 0.25) (layer "F.Cu") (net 5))
 (segment (start 157.525 85.75) (end 161.06 85.75) (width 0.25) (layer "F.Cu") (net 8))
 (segment (start 161.06 85.75) (end 161.8 86.49) (width 0.25) (layer "F.Cu") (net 8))
 (segment (start 152.475 85.25) (end 151.723 85.25) (width 0.25) (layer "F.Cu") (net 9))
 (segment (start 151.723 85.25) (end 149.413 87.56) (width 0.25) (layer "F.Cu") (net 9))
 (segment (start 149.413 87.56) (end 148.2 87.56) (width 0.25) (layer "F.Cu") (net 9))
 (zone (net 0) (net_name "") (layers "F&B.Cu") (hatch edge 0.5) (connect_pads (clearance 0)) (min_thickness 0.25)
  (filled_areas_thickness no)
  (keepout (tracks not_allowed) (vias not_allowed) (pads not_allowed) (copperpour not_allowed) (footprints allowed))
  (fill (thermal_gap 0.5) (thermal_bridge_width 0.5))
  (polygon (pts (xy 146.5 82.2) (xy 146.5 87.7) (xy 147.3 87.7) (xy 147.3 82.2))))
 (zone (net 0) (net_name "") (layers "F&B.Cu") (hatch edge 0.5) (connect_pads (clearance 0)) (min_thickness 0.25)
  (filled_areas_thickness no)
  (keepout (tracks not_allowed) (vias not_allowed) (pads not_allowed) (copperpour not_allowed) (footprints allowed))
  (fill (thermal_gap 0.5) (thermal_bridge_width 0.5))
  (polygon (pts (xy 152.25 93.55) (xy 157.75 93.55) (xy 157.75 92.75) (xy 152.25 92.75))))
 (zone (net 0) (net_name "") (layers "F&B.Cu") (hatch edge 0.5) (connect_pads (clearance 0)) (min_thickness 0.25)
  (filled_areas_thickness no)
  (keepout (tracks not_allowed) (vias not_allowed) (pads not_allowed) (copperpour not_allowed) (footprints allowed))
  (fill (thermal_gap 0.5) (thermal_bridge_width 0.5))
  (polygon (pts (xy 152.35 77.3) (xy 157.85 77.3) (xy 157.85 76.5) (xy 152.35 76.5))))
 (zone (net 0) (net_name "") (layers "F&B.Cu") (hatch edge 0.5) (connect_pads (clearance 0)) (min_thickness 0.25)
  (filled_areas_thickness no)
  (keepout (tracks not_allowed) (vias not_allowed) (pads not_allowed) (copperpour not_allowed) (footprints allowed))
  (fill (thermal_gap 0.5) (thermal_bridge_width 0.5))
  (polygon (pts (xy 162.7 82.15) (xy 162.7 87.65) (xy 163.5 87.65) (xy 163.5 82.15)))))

